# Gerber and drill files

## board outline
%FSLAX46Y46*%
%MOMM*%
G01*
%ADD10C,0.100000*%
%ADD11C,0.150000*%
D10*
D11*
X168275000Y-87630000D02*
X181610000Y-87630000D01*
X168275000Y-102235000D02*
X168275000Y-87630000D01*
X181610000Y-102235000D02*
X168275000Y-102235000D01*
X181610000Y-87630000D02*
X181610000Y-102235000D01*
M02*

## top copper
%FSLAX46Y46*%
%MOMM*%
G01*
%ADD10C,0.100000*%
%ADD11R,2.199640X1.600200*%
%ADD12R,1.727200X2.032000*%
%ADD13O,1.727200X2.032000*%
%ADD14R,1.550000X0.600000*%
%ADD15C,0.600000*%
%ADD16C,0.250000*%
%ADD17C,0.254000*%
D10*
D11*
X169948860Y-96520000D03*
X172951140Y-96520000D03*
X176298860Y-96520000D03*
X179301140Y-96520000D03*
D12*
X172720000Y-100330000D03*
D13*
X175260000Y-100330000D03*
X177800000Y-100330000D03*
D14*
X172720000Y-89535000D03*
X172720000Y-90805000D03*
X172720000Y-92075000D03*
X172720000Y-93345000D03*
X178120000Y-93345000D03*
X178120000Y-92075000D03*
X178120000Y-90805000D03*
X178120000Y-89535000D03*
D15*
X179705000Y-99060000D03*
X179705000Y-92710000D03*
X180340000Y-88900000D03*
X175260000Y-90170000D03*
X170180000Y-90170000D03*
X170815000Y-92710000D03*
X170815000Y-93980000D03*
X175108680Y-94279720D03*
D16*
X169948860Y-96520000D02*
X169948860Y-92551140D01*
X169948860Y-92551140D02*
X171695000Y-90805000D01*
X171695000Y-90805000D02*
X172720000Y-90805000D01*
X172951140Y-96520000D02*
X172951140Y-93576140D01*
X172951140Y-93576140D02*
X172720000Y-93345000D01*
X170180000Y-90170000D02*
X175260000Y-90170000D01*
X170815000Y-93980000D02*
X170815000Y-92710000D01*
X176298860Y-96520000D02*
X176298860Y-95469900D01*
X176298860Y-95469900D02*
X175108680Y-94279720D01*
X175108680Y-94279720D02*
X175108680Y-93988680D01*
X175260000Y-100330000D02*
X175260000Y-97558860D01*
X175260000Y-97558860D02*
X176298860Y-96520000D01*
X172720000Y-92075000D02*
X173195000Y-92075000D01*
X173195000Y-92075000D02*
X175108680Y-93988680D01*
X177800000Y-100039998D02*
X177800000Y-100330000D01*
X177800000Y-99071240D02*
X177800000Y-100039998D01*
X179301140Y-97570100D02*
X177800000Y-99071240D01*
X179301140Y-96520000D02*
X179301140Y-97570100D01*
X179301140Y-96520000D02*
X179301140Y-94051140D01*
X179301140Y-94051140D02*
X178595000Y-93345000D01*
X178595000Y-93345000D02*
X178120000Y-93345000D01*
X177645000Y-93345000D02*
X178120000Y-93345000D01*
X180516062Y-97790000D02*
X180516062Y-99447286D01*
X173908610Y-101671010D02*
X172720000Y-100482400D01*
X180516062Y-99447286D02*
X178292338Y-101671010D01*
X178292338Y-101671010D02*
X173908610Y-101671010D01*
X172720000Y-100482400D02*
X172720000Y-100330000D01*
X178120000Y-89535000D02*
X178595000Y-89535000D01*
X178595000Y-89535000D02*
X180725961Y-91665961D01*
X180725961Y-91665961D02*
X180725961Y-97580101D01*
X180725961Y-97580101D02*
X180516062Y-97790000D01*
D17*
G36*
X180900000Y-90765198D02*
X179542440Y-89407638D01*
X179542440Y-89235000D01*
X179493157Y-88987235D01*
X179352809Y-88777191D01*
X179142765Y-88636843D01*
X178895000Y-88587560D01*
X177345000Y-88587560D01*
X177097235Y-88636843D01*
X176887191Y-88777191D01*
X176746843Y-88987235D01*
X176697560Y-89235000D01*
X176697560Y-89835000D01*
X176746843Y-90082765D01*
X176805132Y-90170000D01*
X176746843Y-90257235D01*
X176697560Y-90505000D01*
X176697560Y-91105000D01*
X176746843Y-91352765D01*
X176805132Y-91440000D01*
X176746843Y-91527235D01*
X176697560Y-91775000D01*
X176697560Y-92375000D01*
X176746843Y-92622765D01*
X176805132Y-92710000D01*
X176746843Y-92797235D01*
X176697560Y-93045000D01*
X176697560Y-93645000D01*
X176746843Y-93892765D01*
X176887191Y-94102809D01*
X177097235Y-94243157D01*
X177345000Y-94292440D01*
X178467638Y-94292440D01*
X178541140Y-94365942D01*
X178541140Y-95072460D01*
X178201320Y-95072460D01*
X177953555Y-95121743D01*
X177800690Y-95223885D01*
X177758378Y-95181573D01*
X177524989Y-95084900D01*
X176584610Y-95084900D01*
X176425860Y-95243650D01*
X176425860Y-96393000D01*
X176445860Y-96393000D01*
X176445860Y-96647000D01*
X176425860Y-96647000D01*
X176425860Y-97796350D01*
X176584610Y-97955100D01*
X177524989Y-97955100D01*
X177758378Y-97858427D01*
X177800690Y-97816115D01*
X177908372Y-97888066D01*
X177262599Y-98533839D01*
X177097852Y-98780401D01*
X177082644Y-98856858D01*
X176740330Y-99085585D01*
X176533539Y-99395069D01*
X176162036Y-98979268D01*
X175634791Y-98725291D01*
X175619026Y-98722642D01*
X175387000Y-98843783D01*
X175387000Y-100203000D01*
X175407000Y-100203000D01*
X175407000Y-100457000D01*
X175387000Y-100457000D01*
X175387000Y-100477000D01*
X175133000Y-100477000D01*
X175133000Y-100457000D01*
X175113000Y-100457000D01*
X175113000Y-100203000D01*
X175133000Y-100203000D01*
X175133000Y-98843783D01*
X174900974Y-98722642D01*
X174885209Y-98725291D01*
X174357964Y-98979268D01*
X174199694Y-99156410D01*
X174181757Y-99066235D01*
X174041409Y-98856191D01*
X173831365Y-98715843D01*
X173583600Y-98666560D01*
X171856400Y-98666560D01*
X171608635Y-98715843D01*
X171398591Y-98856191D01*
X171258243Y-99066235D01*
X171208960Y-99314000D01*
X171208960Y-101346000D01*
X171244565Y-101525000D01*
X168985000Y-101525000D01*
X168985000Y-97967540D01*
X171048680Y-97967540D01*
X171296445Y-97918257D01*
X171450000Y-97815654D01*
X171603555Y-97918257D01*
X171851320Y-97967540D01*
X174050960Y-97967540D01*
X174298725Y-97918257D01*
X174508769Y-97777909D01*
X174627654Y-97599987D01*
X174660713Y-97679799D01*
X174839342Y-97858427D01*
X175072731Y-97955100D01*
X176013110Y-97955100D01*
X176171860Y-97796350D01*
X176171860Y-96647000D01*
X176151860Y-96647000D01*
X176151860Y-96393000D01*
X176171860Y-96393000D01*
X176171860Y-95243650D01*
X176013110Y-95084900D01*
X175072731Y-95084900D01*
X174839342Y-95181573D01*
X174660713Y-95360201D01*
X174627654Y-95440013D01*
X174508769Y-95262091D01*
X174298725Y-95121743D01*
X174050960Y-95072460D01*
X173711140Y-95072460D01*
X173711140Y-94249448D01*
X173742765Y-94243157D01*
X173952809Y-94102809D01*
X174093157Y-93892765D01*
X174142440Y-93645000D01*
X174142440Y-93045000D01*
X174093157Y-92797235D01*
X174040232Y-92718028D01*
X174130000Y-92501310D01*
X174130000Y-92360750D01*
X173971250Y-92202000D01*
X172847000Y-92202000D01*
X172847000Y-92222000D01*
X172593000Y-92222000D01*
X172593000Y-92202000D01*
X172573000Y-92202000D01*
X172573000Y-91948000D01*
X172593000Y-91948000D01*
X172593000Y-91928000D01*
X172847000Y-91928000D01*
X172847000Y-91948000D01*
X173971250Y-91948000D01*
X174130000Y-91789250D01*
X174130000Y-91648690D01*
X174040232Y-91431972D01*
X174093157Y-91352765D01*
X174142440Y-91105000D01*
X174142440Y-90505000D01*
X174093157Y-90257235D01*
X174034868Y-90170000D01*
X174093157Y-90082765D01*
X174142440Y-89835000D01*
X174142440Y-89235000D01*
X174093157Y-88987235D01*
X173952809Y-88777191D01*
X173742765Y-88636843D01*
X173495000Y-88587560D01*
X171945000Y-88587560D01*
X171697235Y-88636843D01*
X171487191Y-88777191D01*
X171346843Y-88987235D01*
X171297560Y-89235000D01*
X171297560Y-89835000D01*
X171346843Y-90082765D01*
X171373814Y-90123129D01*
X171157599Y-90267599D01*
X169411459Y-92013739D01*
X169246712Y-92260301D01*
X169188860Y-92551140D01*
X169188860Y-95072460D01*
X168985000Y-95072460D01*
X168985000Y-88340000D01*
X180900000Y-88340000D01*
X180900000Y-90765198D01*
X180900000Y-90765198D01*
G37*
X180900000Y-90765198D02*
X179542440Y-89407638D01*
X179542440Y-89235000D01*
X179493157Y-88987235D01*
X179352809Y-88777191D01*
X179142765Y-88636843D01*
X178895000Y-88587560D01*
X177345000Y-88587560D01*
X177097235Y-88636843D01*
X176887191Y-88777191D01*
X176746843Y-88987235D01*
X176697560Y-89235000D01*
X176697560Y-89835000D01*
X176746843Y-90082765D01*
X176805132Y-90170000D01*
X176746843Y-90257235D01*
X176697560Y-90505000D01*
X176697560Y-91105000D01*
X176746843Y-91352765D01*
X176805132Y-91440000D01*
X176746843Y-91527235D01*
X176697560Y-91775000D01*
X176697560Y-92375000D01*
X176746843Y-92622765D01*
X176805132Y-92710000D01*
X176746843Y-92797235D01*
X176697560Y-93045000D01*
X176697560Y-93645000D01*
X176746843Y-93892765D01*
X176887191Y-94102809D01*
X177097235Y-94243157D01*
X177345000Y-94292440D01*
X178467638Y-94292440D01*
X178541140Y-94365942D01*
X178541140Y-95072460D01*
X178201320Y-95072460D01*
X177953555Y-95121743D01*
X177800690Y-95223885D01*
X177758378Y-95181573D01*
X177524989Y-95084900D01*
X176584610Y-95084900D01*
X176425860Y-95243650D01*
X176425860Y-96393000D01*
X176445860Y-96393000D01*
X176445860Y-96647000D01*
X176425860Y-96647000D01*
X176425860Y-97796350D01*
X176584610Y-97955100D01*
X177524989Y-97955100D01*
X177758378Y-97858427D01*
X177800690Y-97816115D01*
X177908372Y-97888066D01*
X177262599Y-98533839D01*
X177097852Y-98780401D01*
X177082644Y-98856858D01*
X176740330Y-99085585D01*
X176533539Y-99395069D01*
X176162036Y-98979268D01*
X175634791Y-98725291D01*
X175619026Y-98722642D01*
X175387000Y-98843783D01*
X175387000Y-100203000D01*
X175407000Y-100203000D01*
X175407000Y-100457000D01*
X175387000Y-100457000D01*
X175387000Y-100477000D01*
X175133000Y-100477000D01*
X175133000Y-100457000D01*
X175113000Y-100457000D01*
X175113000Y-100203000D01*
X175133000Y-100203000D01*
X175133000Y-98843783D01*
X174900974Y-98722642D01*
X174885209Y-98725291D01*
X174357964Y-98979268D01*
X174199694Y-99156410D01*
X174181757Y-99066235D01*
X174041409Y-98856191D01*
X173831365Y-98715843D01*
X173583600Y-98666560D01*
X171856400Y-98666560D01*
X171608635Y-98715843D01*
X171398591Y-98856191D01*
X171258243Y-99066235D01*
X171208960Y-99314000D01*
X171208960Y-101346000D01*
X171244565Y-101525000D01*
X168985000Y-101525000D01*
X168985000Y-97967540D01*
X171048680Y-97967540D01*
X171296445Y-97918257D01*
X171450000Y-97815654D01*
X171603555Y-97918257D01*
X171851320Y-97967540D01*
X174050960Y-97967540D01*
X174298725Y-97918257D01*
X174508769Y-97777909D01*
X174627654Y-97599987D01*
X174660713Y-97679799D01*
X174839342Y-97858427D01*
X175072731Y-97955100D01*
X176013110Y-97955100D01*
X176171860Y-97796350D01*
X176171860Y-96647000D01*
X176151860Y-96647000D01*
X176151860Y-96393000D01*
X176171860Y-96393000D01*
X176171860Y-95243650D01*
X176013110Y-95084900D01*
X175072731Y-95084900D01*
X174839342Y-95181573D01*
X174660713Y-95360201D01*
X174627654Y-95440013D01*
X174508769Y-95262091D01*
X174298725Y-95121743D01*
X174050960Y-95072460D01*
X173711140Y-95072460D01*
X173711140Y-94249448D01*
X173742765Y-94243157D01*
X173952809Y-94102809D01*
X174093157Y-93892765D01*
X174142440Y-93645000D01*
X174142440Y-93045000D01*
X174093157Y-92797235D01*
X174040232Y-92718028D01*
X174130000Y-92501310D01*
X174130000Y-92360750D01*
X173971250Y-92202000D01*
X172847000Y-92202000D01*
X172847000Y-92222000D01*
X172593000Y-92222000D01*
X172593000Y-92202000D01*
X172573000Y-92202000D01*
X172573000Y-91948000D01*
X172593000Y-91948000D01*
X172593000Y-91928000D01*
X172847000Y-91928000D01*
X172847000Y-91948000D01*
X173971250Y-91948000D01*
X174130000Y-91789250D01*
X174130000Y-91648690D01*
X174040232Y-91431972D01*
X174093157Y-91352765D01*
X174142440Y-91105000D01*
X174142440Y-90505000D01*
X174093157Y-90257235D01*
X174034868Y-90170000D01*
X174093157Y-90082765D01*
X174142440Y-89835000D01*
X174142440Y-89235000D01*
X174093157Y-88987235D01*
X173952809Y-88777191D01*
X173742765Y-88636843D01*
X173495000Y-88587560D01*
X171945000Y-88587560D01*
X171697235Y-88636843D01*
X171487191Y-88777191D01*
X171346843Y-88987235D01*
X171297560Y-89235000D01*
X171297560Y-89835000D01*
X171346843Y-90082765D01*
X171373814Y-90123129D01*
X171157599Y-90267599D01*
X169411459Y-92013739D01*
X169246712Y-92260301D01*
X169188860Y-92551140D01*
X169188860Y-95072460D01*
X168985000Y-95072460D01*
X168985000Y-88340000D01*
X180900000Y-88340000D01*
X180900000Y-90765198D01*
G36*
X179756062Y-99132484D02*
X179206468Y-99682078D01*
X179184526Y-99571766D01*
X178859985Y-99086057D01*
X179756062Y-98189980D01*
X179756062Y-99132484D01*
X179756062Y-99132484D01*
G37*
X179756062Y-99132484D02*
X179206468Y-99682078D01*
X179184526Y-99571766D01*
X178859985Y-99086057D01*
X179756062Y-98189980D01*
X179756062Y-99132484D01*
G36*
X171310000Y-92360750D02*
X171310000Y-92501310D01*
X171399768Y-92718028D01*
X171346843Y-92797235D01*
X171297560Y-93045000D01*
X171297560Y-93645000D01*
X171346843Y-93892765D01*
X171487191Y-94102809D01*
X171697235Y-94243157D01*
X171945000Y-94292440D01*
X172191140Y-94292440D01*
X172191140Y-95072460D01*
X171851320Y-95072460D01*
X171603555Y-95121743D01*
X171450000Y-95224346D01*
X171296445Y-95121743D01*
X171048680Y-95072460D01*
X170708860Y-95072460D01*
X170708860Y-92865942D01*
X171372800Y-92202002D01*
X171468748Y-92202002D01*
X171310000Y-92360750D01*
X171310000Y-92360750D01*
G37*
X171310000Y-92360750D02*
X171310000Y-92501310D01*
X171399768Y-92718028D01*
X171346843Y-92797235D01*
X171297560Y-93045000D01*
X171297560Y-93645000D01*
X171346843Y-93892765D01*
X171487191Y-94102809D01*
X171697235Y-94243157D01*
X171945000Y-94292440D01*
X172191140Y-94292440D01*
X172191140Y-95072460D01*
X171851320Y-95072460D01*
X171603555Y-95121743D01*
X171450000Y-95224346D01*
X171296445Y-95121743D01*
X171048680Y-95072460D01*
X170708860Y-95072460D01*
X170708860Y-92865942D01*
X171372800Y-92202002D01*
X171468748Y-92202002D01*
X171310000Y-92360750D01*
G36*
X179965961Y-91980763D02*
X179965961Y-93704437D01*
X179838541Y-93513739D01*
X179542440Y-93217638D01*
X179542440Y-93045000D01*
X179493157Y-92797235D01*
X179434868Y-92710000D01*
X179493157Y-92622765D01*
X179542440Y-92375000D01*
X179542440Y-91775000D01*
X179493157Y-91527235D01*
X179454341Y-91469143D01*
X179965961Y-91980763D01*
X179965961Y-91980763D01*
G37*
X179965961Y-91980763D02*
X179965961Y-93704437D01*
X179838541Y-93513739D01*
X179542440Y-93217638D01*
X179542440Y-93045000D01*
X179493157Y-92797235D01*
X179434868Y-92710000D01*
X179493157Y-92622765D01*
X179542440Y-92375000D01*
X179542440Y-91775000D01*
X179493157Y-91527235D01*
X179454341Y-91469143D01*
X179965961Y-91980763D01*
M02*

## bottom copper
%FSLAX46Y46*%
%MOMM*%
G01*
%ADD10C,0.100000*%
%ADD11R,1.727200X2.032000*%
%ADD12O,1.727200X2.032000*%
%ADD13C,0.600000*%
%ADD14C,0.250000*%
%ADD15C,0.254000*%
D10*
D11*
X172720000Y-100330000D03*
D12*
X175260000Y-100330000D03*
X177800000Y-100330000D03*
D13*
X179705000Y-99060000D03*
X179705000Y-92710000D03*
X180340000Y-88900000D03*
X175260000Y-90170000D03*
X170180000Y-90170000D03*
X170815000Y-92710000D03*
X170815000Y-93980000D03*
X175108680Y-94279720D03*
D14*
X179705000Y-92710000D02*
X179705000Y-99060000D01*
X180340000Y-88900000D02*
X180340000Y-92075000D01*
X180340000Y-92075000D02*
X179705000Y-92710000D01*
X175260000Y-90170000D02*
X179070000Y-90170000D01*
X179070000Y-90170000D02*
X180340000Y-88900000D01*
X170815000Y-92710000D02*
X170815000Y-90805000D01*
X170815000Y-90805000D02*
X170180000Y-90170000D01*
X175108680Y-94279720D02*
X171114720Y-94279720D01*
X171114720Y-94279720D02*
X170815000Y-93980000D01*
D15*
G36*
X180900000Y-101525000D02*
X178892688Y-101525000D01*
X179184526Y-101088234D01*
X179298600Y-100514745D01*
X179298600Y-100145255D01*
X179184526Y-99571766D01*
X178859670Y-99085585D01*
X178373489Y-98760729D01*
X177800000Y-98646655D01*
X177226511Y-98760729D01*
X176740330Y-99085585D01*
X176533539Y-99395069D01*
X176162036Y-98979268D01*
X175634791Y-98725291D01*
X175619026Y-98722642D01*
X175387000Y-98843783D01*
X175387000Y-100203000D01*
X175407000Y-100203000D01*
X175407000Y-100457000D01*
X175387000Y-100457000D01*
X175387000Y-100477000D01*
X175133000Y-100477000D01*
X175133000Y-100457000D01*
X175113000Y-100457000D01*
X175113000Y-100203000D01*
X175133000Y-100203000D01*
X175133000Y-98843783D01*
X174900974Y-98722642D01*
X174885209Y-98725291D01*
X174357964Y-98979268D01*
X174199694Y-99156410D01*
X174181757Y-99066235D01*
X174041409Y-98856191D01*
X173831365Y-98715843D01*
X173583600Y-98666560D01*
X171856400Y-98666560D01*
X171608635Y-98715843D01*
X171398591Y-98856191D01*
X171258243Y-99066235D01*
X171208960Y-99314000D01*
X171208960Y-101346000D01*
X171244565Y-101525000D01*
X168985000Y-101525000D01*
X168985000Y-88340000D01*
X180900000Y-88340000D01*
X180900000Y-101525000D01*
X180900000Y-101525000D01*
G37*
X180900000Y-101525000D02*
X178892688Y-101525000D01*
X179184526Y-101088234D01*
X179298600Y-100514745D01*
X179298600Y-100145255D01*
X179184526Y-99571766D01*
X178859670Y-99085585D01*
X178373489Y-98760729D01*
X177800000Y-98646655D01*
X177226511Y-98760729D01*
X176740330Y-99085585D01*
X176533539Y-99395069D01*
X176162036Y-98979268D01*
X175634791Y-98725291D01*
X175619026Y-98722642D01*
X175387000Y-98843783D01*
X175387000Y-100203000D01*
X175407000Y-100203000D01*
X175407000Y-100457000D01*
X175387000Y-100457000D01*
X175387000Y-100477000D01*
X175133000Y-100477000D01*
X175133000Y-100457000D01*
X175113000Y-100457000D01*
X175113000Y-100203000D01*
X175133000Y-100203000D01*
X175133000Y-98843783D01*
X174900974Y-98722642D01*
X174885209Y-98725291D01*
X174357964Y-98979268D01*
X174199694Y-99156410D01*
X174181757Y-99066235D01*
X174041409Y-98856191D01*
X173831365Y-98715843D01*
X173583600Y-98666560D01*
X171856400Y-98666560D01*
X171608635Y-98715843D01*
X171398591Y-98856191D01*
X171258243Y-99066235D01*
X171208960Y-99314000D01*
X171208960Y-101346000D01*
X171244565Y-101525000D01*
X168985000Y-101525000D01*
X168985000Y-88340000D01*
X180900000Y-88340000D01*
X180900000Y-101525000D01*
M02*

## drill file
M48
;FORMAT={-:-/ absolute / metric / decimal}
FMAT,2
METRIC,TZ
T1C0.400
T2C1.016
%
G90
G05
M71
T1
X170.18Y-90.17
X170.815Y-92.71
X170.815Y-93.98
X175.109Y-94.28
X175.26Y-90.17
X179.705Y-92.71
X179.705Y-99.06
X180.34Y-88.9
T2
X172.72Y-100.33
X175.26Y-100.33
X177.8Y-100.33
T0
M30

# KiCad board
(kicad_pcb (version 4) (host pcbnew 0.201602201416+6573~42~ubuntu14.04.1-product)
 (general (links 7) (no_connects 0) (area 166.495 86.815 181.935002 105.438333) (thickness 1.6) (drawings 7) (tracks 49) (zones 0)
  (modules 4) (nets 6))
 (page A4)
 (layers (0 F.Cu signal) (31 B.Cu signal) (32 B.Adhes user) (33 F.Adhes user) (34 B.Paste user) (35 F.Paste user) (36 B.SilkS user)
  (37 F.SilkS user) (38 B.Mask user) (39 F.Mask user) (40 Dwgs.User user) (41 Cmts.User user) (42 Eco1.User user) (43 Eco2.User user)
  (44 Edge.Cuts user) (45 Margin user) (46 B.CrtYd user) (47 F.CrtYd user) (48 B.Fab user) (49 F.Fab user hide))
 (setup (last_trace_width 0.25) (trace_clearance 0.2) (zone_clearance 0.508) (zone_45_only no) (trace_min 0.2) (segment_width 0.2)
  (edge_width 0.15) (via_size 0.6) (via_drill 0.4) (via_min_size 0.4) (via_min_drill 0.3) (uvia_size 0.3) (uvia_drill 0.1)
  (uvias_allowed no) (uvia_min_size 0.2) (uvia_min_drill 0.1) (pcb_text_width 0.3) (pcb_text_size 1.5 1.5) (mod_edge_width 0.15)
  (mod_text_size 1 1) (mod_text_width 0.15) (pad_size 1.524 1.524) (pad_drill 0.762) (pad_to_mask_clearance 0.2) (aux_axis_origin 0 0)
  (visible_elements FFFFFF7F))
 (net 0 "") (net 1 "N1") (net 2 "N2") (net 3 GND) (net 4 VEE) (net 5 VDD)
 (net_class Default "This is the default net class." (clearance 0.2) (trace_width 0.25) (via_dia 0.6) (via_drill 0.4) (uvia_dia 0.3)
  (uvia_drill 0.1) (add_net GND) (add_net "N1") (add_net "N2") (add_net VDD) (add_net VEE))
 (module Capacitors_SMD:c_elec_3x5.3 (layer F.Cu) (at 171.45 96.52 180)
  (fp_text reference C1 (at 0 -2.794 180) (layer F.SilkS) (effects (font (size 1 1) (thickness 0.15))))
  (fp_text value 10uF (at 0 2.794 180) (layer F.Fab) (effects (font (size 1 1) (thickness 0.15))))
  (pad 1 smd rect (at 1.50114 0 180) (size 2.19964 1.6002) (layers F.Cu F.Paste F.Mask) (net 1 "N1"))
  (pad 2 smd rect (at -1.50114 0 180) (size 2.19964 1.6002) (layers F.Cu F.Paste F.Mask) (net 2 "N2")))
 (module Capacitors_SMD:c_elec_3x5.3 (layer F.Cu) (at 177.8 96.52 180)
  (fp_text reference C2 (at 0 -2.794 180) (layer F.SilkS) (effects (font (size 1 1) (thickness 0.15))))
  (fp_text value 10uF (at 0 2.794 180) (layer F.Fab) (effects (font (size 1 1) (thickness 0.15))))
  (pad 1 smd rect (at 1.50114 0 180) (size 2.19964 1.6002) (layers F.Cu F.Paste F.Mask) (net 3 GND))
  (pad 2 smd rect (at -1.50114 0 180) (size 2.19964 1.6002) (layers F.Cu F.Paste F.Mask) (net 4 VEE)))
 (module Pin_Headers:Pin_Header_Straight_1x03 (layer F.Cu) (at 172.72 100.33 90)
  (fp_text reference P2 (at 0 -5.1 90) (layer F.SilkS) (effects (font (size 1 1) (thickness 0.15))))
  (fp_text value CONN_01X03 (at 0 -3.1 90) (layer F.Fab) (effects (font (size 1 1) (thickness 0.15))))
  (pad 1 thru_hole rect (at 0 0 90) (size 2.032 1.7272) (drill 1.016) (layers *.Cu *.Mask F.SilkS) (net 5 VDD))
  (pad 2 thru_hole oval (at 0 2.54 90) (size 2.032 1.7272) (drill 1.016) (layers *.Cu *.Mask F.SilkS) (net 3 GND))
  (pad 3 thru_hole oval (at 0 5.08 90) (size 2.032 1.7272) (drill 1.016) (layers *.Cu *.Mask F.SilkS) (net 4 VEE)))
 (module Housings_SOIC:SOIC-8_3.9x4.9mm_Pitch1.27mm (layer F.Cu) (at 175.42 91.44)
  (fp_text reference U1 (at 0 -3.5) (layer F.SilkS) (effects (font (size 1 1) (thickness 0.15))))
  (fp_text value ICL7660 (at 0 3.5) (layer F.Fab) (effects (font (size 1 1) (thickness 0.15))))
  (pad 1 smd rect (at -2.7 -1.905) (size 1.55 0.6) (layers F.Cu F.Paste F.Mask))
  (pad 2 smd rect (at -2.7 -0.635) (size 1.55 0.6) (layers F.Cu F.Paste F.Mask) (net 1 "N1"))
  (pad 3 smd rect (at -2.7 0.635) (size 1.55 0.6) (layers F.Cu F.Paste F.Mask) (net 3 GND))
  (pad 4 smd rect (at -2.7 1.905) (size 1.55 0.6) (layers F.Cu F.Paste F.Mask) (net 2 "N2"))
  (pad 5 smd rect (at 2.7 1.905) (size 1.55 0.6) (layers F.Cu F.Paste F.Mask) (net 4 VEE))
  (pad 6 smd rect (at 2.7 0.635) (size 1.55 0.6) (layers F.Cu F.Paste F.Mask))
  (pad 7 smd rect (at 2.7 -0.635) (size 1.55 0.6) (layers F.Cu F.Paste F.Mask))
  (pad 8 smd rect (at 2.7 -1.905) (size 1.55 0.6) (layers F.Cu F.Paste F.Mask) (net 5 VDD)))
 (gr_line (start 168.275 87.63) (end 181.61 87.63) (layer Edge.Cuts) (width 0.15))
 (gr_line (start 168.275 102.235) (end 168.275 87.63) (layer Edge.Cuts) (width 0.15))
 (gr_line (start 181.61 102.235) (end 168.275 102.235) (layer Edge.Cuts) (width 0.15))
 (gr_line (start 181.61 87.63) (end 181.61 102.235) (layer Edge.Cuts) (width 0.15))
 (segment (start 181.61 87.63) (end 181.61 101.6) (width 0.25) (layer Dwgs.User) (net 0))
 (segment (start 169.94886 96.52) (end 169.94886 92.55114) (width 0.25) (layer F.Cu) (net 1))
 (segment (start 169.94886 92.55114) (end 171.695 90.805) (width 0.25) (layer F.Cu) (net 1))
 (segment (start 171.695 90.805) (end 172.72 90.805) (width 0.25) (layer F.Cu) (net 1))
 (segment (start 172.95114 96.52) (end 172.95114 93.57614) (width 0.25) (layer F.Cu) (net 2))
 (segment (start 172.95114 93.57614) (end 172.72 93.345) (width 0.25) (layer F.Cu) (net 2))
 (via (at 179.705 99.06) (size 0.6) (drill 0.4) (layers F.Cu B.Cu) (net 3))
 (segment (start 179.705 92.71) (end 179.705 99.06) (width 0.25) (layer B.Cu) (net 3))
 (segment (start 180.34 88.9) (end 180.34 92.075) (width 0.25) (layer B.Cu) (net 3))
 (segment (start 180.34 92.075) (end 179.705 92.71) (width 0.25) (layer B.Cu) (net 3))
 (via (at 179.705 92.71) (size 0.6) (drill 0.4) (layers F.Cu B.Cu) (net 3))
 (segment (start 175.26 90.17) (end 179.07 90.17) (width 0.25) (layer B.Cu) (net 3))
 (segment (start 179.07 90.17) (end 180.34 88.9) (width 0.25) (layer B.Cu) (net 3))
 (via (at 180.34 88.9) (size 0.6) (drill 0.4) (layers F.Cu B.Cu) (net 3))
 (segment (start 170.18 90.17) (end 175.26 90.17) (width 0.25) (layer F.Cu) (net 3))
 (via (at 175.26 90.17) (size 0.6) (drill 0.4) (layers F.Cu B.Cu) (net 3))
 (segment (start 170.815 92.71) (end 170.815 90.805) (width 0.25) (layer B.Cu) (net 3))
 (segment (start 170.815 90.805) (end 170.18 90.17) (width 0.25) (layer B.Cu) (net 3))
 (via (at 170.18 90.17) (size 0.6) (drill 0.4) (layers F.Cu B.Cu) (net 3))
 (segment (start 170.815 93.98) (end 170.815 92.71) (width 0.25) (layer F.Cu) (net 3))
 (via (at 170.815 92.71) (size 0.6) (drill 0.4) (layers F.Cu B.Cu) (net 3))
 (segment (start 175.10868 94.27972) (end 171.11472 94.27972) (width 0.25) (layer B.Cu) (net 3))
 (segment (start 171.11472 94.27972) (end 170.815 93.98) (width 0.25) (layer B.Cu) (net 3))
 (via (at 170.815 93.98) (size 0.6) (drill 0.4) (layers F.Cu B.Cu) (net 3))
 (segment (start 176.29886 96.52) (end 176.29886 95.4699) (width 0.25) (layer F.Cu) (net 3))
 (segment (start 176.29886 95.4699) (end 175.10868 94.27972) (width 0.25) (layer F.Cu) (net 3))
 (via (at 175.10868 94.27972) (size 0.6) (drill 0.4) (layers F.Cu B.Cu) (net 3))
 (segment (start 175.10868 94.27972) (end 175.10868 93.98868) (width 0.25) (layer F.Cu) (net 3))
 (segment (start 175.26 100.33) (end 175.26 97.55886) (width 0.25) (layer F.Cu) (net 3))
 (segment (start 175.26 97.55886) (end 176.29886 96.52) (width 0.25) (layer F.Cu) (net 3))
 (segment (start 172.72 92.075) (end 173.195 92.075) (width 0.25) (layer F.Cu) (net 3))
 (segment (start 173.195 92.075) (end 175.10868 93.98868) (width 0.25) (layer F.Cu) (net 3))
 (segment (start 177.8 100.039998) (end 177.8 100.33) (width 0.25) (layer F.Cu) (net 4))
 (segment (start 177.8 99.07124) (end 177.8 100.039998) (width 0.25) (layer F.Cu) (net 4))
 (segment (start 179.30114 97.5701) (end 177.8 99.07124) (width 0.25) (layer F.Cu) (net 4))
 (segment (start 179.30114 96.52) (end 179.30114 97.5701) (width 0.25) (layer F.Cu) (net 4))
 (segment (start 179.30114 96.52) (end 179.30114 94.05114) (width 0.25) (layer F.Cu) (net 4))
 (segment (start 179.30114 94.05114) (end 178.595 93.345) (width 0.25) (layer F.Cu) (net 4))
 (segment (start 178.595 93.345) (end 178.12 93.345) (width 0.25) (layer F.Cu) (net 4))
 (segment (start 177.645 93.345) (end 178.12 93.345) (width 0.25) (layer F.Cu) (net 4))
 (segment (start 180.516062 97.79) (end 180.516062 99.447286) (width 0.25) (layer F.Cu) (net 5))
 (segment (start 173.90861 101.67101) (end 172.72 100.4824) (width 0.25) (layer F.Cu) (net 5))
 (segment (start 180.516062 99.447286) (end 178.292338 101.67101) (width 0.25) (layer F.Cu) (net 5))
 (segment (start 178.292338 101.67101) (end 173.90861 101.67101) (width 0.25) (layer F.Cu) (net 5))
 (segment (start 172.72 100.4824) (end 172.72 100.33) (width 0.25) (layer F.Cu) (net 5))
 (segment (start 178.12 89.535) (end 178.595 89.535) (width 0.25) (layer F.Cu) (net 5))
 (segment (start 178.595 89.535) (end 180.725961 91.665961) (width 0.25) (layer F.Cu) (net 5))
 (segment (start 180.725961 91.665961) (end 180.725961 97.580101) (width 0.25) (layer F.Cu) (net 5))
 (segment (start 180.725961 97.580101) (end 180.516062 97.79) (width 0.25) (layer F.Cu) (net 5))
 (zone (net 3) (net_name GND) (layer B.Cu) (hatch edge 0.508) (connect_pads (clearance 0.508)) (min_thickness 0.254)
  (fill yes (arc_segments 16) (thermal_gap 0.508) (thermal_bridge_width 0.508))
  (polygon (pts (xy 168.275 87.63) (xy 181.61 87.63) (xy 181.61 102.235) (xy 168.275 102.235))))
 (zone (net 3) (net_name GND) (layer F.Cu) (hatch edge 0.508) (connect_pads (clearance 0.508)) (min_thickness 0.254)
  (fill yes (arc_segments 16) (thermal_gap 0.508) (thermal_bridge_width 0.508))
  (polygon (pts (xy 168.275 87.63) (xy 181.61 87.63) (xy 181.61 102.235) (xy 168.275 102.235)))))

